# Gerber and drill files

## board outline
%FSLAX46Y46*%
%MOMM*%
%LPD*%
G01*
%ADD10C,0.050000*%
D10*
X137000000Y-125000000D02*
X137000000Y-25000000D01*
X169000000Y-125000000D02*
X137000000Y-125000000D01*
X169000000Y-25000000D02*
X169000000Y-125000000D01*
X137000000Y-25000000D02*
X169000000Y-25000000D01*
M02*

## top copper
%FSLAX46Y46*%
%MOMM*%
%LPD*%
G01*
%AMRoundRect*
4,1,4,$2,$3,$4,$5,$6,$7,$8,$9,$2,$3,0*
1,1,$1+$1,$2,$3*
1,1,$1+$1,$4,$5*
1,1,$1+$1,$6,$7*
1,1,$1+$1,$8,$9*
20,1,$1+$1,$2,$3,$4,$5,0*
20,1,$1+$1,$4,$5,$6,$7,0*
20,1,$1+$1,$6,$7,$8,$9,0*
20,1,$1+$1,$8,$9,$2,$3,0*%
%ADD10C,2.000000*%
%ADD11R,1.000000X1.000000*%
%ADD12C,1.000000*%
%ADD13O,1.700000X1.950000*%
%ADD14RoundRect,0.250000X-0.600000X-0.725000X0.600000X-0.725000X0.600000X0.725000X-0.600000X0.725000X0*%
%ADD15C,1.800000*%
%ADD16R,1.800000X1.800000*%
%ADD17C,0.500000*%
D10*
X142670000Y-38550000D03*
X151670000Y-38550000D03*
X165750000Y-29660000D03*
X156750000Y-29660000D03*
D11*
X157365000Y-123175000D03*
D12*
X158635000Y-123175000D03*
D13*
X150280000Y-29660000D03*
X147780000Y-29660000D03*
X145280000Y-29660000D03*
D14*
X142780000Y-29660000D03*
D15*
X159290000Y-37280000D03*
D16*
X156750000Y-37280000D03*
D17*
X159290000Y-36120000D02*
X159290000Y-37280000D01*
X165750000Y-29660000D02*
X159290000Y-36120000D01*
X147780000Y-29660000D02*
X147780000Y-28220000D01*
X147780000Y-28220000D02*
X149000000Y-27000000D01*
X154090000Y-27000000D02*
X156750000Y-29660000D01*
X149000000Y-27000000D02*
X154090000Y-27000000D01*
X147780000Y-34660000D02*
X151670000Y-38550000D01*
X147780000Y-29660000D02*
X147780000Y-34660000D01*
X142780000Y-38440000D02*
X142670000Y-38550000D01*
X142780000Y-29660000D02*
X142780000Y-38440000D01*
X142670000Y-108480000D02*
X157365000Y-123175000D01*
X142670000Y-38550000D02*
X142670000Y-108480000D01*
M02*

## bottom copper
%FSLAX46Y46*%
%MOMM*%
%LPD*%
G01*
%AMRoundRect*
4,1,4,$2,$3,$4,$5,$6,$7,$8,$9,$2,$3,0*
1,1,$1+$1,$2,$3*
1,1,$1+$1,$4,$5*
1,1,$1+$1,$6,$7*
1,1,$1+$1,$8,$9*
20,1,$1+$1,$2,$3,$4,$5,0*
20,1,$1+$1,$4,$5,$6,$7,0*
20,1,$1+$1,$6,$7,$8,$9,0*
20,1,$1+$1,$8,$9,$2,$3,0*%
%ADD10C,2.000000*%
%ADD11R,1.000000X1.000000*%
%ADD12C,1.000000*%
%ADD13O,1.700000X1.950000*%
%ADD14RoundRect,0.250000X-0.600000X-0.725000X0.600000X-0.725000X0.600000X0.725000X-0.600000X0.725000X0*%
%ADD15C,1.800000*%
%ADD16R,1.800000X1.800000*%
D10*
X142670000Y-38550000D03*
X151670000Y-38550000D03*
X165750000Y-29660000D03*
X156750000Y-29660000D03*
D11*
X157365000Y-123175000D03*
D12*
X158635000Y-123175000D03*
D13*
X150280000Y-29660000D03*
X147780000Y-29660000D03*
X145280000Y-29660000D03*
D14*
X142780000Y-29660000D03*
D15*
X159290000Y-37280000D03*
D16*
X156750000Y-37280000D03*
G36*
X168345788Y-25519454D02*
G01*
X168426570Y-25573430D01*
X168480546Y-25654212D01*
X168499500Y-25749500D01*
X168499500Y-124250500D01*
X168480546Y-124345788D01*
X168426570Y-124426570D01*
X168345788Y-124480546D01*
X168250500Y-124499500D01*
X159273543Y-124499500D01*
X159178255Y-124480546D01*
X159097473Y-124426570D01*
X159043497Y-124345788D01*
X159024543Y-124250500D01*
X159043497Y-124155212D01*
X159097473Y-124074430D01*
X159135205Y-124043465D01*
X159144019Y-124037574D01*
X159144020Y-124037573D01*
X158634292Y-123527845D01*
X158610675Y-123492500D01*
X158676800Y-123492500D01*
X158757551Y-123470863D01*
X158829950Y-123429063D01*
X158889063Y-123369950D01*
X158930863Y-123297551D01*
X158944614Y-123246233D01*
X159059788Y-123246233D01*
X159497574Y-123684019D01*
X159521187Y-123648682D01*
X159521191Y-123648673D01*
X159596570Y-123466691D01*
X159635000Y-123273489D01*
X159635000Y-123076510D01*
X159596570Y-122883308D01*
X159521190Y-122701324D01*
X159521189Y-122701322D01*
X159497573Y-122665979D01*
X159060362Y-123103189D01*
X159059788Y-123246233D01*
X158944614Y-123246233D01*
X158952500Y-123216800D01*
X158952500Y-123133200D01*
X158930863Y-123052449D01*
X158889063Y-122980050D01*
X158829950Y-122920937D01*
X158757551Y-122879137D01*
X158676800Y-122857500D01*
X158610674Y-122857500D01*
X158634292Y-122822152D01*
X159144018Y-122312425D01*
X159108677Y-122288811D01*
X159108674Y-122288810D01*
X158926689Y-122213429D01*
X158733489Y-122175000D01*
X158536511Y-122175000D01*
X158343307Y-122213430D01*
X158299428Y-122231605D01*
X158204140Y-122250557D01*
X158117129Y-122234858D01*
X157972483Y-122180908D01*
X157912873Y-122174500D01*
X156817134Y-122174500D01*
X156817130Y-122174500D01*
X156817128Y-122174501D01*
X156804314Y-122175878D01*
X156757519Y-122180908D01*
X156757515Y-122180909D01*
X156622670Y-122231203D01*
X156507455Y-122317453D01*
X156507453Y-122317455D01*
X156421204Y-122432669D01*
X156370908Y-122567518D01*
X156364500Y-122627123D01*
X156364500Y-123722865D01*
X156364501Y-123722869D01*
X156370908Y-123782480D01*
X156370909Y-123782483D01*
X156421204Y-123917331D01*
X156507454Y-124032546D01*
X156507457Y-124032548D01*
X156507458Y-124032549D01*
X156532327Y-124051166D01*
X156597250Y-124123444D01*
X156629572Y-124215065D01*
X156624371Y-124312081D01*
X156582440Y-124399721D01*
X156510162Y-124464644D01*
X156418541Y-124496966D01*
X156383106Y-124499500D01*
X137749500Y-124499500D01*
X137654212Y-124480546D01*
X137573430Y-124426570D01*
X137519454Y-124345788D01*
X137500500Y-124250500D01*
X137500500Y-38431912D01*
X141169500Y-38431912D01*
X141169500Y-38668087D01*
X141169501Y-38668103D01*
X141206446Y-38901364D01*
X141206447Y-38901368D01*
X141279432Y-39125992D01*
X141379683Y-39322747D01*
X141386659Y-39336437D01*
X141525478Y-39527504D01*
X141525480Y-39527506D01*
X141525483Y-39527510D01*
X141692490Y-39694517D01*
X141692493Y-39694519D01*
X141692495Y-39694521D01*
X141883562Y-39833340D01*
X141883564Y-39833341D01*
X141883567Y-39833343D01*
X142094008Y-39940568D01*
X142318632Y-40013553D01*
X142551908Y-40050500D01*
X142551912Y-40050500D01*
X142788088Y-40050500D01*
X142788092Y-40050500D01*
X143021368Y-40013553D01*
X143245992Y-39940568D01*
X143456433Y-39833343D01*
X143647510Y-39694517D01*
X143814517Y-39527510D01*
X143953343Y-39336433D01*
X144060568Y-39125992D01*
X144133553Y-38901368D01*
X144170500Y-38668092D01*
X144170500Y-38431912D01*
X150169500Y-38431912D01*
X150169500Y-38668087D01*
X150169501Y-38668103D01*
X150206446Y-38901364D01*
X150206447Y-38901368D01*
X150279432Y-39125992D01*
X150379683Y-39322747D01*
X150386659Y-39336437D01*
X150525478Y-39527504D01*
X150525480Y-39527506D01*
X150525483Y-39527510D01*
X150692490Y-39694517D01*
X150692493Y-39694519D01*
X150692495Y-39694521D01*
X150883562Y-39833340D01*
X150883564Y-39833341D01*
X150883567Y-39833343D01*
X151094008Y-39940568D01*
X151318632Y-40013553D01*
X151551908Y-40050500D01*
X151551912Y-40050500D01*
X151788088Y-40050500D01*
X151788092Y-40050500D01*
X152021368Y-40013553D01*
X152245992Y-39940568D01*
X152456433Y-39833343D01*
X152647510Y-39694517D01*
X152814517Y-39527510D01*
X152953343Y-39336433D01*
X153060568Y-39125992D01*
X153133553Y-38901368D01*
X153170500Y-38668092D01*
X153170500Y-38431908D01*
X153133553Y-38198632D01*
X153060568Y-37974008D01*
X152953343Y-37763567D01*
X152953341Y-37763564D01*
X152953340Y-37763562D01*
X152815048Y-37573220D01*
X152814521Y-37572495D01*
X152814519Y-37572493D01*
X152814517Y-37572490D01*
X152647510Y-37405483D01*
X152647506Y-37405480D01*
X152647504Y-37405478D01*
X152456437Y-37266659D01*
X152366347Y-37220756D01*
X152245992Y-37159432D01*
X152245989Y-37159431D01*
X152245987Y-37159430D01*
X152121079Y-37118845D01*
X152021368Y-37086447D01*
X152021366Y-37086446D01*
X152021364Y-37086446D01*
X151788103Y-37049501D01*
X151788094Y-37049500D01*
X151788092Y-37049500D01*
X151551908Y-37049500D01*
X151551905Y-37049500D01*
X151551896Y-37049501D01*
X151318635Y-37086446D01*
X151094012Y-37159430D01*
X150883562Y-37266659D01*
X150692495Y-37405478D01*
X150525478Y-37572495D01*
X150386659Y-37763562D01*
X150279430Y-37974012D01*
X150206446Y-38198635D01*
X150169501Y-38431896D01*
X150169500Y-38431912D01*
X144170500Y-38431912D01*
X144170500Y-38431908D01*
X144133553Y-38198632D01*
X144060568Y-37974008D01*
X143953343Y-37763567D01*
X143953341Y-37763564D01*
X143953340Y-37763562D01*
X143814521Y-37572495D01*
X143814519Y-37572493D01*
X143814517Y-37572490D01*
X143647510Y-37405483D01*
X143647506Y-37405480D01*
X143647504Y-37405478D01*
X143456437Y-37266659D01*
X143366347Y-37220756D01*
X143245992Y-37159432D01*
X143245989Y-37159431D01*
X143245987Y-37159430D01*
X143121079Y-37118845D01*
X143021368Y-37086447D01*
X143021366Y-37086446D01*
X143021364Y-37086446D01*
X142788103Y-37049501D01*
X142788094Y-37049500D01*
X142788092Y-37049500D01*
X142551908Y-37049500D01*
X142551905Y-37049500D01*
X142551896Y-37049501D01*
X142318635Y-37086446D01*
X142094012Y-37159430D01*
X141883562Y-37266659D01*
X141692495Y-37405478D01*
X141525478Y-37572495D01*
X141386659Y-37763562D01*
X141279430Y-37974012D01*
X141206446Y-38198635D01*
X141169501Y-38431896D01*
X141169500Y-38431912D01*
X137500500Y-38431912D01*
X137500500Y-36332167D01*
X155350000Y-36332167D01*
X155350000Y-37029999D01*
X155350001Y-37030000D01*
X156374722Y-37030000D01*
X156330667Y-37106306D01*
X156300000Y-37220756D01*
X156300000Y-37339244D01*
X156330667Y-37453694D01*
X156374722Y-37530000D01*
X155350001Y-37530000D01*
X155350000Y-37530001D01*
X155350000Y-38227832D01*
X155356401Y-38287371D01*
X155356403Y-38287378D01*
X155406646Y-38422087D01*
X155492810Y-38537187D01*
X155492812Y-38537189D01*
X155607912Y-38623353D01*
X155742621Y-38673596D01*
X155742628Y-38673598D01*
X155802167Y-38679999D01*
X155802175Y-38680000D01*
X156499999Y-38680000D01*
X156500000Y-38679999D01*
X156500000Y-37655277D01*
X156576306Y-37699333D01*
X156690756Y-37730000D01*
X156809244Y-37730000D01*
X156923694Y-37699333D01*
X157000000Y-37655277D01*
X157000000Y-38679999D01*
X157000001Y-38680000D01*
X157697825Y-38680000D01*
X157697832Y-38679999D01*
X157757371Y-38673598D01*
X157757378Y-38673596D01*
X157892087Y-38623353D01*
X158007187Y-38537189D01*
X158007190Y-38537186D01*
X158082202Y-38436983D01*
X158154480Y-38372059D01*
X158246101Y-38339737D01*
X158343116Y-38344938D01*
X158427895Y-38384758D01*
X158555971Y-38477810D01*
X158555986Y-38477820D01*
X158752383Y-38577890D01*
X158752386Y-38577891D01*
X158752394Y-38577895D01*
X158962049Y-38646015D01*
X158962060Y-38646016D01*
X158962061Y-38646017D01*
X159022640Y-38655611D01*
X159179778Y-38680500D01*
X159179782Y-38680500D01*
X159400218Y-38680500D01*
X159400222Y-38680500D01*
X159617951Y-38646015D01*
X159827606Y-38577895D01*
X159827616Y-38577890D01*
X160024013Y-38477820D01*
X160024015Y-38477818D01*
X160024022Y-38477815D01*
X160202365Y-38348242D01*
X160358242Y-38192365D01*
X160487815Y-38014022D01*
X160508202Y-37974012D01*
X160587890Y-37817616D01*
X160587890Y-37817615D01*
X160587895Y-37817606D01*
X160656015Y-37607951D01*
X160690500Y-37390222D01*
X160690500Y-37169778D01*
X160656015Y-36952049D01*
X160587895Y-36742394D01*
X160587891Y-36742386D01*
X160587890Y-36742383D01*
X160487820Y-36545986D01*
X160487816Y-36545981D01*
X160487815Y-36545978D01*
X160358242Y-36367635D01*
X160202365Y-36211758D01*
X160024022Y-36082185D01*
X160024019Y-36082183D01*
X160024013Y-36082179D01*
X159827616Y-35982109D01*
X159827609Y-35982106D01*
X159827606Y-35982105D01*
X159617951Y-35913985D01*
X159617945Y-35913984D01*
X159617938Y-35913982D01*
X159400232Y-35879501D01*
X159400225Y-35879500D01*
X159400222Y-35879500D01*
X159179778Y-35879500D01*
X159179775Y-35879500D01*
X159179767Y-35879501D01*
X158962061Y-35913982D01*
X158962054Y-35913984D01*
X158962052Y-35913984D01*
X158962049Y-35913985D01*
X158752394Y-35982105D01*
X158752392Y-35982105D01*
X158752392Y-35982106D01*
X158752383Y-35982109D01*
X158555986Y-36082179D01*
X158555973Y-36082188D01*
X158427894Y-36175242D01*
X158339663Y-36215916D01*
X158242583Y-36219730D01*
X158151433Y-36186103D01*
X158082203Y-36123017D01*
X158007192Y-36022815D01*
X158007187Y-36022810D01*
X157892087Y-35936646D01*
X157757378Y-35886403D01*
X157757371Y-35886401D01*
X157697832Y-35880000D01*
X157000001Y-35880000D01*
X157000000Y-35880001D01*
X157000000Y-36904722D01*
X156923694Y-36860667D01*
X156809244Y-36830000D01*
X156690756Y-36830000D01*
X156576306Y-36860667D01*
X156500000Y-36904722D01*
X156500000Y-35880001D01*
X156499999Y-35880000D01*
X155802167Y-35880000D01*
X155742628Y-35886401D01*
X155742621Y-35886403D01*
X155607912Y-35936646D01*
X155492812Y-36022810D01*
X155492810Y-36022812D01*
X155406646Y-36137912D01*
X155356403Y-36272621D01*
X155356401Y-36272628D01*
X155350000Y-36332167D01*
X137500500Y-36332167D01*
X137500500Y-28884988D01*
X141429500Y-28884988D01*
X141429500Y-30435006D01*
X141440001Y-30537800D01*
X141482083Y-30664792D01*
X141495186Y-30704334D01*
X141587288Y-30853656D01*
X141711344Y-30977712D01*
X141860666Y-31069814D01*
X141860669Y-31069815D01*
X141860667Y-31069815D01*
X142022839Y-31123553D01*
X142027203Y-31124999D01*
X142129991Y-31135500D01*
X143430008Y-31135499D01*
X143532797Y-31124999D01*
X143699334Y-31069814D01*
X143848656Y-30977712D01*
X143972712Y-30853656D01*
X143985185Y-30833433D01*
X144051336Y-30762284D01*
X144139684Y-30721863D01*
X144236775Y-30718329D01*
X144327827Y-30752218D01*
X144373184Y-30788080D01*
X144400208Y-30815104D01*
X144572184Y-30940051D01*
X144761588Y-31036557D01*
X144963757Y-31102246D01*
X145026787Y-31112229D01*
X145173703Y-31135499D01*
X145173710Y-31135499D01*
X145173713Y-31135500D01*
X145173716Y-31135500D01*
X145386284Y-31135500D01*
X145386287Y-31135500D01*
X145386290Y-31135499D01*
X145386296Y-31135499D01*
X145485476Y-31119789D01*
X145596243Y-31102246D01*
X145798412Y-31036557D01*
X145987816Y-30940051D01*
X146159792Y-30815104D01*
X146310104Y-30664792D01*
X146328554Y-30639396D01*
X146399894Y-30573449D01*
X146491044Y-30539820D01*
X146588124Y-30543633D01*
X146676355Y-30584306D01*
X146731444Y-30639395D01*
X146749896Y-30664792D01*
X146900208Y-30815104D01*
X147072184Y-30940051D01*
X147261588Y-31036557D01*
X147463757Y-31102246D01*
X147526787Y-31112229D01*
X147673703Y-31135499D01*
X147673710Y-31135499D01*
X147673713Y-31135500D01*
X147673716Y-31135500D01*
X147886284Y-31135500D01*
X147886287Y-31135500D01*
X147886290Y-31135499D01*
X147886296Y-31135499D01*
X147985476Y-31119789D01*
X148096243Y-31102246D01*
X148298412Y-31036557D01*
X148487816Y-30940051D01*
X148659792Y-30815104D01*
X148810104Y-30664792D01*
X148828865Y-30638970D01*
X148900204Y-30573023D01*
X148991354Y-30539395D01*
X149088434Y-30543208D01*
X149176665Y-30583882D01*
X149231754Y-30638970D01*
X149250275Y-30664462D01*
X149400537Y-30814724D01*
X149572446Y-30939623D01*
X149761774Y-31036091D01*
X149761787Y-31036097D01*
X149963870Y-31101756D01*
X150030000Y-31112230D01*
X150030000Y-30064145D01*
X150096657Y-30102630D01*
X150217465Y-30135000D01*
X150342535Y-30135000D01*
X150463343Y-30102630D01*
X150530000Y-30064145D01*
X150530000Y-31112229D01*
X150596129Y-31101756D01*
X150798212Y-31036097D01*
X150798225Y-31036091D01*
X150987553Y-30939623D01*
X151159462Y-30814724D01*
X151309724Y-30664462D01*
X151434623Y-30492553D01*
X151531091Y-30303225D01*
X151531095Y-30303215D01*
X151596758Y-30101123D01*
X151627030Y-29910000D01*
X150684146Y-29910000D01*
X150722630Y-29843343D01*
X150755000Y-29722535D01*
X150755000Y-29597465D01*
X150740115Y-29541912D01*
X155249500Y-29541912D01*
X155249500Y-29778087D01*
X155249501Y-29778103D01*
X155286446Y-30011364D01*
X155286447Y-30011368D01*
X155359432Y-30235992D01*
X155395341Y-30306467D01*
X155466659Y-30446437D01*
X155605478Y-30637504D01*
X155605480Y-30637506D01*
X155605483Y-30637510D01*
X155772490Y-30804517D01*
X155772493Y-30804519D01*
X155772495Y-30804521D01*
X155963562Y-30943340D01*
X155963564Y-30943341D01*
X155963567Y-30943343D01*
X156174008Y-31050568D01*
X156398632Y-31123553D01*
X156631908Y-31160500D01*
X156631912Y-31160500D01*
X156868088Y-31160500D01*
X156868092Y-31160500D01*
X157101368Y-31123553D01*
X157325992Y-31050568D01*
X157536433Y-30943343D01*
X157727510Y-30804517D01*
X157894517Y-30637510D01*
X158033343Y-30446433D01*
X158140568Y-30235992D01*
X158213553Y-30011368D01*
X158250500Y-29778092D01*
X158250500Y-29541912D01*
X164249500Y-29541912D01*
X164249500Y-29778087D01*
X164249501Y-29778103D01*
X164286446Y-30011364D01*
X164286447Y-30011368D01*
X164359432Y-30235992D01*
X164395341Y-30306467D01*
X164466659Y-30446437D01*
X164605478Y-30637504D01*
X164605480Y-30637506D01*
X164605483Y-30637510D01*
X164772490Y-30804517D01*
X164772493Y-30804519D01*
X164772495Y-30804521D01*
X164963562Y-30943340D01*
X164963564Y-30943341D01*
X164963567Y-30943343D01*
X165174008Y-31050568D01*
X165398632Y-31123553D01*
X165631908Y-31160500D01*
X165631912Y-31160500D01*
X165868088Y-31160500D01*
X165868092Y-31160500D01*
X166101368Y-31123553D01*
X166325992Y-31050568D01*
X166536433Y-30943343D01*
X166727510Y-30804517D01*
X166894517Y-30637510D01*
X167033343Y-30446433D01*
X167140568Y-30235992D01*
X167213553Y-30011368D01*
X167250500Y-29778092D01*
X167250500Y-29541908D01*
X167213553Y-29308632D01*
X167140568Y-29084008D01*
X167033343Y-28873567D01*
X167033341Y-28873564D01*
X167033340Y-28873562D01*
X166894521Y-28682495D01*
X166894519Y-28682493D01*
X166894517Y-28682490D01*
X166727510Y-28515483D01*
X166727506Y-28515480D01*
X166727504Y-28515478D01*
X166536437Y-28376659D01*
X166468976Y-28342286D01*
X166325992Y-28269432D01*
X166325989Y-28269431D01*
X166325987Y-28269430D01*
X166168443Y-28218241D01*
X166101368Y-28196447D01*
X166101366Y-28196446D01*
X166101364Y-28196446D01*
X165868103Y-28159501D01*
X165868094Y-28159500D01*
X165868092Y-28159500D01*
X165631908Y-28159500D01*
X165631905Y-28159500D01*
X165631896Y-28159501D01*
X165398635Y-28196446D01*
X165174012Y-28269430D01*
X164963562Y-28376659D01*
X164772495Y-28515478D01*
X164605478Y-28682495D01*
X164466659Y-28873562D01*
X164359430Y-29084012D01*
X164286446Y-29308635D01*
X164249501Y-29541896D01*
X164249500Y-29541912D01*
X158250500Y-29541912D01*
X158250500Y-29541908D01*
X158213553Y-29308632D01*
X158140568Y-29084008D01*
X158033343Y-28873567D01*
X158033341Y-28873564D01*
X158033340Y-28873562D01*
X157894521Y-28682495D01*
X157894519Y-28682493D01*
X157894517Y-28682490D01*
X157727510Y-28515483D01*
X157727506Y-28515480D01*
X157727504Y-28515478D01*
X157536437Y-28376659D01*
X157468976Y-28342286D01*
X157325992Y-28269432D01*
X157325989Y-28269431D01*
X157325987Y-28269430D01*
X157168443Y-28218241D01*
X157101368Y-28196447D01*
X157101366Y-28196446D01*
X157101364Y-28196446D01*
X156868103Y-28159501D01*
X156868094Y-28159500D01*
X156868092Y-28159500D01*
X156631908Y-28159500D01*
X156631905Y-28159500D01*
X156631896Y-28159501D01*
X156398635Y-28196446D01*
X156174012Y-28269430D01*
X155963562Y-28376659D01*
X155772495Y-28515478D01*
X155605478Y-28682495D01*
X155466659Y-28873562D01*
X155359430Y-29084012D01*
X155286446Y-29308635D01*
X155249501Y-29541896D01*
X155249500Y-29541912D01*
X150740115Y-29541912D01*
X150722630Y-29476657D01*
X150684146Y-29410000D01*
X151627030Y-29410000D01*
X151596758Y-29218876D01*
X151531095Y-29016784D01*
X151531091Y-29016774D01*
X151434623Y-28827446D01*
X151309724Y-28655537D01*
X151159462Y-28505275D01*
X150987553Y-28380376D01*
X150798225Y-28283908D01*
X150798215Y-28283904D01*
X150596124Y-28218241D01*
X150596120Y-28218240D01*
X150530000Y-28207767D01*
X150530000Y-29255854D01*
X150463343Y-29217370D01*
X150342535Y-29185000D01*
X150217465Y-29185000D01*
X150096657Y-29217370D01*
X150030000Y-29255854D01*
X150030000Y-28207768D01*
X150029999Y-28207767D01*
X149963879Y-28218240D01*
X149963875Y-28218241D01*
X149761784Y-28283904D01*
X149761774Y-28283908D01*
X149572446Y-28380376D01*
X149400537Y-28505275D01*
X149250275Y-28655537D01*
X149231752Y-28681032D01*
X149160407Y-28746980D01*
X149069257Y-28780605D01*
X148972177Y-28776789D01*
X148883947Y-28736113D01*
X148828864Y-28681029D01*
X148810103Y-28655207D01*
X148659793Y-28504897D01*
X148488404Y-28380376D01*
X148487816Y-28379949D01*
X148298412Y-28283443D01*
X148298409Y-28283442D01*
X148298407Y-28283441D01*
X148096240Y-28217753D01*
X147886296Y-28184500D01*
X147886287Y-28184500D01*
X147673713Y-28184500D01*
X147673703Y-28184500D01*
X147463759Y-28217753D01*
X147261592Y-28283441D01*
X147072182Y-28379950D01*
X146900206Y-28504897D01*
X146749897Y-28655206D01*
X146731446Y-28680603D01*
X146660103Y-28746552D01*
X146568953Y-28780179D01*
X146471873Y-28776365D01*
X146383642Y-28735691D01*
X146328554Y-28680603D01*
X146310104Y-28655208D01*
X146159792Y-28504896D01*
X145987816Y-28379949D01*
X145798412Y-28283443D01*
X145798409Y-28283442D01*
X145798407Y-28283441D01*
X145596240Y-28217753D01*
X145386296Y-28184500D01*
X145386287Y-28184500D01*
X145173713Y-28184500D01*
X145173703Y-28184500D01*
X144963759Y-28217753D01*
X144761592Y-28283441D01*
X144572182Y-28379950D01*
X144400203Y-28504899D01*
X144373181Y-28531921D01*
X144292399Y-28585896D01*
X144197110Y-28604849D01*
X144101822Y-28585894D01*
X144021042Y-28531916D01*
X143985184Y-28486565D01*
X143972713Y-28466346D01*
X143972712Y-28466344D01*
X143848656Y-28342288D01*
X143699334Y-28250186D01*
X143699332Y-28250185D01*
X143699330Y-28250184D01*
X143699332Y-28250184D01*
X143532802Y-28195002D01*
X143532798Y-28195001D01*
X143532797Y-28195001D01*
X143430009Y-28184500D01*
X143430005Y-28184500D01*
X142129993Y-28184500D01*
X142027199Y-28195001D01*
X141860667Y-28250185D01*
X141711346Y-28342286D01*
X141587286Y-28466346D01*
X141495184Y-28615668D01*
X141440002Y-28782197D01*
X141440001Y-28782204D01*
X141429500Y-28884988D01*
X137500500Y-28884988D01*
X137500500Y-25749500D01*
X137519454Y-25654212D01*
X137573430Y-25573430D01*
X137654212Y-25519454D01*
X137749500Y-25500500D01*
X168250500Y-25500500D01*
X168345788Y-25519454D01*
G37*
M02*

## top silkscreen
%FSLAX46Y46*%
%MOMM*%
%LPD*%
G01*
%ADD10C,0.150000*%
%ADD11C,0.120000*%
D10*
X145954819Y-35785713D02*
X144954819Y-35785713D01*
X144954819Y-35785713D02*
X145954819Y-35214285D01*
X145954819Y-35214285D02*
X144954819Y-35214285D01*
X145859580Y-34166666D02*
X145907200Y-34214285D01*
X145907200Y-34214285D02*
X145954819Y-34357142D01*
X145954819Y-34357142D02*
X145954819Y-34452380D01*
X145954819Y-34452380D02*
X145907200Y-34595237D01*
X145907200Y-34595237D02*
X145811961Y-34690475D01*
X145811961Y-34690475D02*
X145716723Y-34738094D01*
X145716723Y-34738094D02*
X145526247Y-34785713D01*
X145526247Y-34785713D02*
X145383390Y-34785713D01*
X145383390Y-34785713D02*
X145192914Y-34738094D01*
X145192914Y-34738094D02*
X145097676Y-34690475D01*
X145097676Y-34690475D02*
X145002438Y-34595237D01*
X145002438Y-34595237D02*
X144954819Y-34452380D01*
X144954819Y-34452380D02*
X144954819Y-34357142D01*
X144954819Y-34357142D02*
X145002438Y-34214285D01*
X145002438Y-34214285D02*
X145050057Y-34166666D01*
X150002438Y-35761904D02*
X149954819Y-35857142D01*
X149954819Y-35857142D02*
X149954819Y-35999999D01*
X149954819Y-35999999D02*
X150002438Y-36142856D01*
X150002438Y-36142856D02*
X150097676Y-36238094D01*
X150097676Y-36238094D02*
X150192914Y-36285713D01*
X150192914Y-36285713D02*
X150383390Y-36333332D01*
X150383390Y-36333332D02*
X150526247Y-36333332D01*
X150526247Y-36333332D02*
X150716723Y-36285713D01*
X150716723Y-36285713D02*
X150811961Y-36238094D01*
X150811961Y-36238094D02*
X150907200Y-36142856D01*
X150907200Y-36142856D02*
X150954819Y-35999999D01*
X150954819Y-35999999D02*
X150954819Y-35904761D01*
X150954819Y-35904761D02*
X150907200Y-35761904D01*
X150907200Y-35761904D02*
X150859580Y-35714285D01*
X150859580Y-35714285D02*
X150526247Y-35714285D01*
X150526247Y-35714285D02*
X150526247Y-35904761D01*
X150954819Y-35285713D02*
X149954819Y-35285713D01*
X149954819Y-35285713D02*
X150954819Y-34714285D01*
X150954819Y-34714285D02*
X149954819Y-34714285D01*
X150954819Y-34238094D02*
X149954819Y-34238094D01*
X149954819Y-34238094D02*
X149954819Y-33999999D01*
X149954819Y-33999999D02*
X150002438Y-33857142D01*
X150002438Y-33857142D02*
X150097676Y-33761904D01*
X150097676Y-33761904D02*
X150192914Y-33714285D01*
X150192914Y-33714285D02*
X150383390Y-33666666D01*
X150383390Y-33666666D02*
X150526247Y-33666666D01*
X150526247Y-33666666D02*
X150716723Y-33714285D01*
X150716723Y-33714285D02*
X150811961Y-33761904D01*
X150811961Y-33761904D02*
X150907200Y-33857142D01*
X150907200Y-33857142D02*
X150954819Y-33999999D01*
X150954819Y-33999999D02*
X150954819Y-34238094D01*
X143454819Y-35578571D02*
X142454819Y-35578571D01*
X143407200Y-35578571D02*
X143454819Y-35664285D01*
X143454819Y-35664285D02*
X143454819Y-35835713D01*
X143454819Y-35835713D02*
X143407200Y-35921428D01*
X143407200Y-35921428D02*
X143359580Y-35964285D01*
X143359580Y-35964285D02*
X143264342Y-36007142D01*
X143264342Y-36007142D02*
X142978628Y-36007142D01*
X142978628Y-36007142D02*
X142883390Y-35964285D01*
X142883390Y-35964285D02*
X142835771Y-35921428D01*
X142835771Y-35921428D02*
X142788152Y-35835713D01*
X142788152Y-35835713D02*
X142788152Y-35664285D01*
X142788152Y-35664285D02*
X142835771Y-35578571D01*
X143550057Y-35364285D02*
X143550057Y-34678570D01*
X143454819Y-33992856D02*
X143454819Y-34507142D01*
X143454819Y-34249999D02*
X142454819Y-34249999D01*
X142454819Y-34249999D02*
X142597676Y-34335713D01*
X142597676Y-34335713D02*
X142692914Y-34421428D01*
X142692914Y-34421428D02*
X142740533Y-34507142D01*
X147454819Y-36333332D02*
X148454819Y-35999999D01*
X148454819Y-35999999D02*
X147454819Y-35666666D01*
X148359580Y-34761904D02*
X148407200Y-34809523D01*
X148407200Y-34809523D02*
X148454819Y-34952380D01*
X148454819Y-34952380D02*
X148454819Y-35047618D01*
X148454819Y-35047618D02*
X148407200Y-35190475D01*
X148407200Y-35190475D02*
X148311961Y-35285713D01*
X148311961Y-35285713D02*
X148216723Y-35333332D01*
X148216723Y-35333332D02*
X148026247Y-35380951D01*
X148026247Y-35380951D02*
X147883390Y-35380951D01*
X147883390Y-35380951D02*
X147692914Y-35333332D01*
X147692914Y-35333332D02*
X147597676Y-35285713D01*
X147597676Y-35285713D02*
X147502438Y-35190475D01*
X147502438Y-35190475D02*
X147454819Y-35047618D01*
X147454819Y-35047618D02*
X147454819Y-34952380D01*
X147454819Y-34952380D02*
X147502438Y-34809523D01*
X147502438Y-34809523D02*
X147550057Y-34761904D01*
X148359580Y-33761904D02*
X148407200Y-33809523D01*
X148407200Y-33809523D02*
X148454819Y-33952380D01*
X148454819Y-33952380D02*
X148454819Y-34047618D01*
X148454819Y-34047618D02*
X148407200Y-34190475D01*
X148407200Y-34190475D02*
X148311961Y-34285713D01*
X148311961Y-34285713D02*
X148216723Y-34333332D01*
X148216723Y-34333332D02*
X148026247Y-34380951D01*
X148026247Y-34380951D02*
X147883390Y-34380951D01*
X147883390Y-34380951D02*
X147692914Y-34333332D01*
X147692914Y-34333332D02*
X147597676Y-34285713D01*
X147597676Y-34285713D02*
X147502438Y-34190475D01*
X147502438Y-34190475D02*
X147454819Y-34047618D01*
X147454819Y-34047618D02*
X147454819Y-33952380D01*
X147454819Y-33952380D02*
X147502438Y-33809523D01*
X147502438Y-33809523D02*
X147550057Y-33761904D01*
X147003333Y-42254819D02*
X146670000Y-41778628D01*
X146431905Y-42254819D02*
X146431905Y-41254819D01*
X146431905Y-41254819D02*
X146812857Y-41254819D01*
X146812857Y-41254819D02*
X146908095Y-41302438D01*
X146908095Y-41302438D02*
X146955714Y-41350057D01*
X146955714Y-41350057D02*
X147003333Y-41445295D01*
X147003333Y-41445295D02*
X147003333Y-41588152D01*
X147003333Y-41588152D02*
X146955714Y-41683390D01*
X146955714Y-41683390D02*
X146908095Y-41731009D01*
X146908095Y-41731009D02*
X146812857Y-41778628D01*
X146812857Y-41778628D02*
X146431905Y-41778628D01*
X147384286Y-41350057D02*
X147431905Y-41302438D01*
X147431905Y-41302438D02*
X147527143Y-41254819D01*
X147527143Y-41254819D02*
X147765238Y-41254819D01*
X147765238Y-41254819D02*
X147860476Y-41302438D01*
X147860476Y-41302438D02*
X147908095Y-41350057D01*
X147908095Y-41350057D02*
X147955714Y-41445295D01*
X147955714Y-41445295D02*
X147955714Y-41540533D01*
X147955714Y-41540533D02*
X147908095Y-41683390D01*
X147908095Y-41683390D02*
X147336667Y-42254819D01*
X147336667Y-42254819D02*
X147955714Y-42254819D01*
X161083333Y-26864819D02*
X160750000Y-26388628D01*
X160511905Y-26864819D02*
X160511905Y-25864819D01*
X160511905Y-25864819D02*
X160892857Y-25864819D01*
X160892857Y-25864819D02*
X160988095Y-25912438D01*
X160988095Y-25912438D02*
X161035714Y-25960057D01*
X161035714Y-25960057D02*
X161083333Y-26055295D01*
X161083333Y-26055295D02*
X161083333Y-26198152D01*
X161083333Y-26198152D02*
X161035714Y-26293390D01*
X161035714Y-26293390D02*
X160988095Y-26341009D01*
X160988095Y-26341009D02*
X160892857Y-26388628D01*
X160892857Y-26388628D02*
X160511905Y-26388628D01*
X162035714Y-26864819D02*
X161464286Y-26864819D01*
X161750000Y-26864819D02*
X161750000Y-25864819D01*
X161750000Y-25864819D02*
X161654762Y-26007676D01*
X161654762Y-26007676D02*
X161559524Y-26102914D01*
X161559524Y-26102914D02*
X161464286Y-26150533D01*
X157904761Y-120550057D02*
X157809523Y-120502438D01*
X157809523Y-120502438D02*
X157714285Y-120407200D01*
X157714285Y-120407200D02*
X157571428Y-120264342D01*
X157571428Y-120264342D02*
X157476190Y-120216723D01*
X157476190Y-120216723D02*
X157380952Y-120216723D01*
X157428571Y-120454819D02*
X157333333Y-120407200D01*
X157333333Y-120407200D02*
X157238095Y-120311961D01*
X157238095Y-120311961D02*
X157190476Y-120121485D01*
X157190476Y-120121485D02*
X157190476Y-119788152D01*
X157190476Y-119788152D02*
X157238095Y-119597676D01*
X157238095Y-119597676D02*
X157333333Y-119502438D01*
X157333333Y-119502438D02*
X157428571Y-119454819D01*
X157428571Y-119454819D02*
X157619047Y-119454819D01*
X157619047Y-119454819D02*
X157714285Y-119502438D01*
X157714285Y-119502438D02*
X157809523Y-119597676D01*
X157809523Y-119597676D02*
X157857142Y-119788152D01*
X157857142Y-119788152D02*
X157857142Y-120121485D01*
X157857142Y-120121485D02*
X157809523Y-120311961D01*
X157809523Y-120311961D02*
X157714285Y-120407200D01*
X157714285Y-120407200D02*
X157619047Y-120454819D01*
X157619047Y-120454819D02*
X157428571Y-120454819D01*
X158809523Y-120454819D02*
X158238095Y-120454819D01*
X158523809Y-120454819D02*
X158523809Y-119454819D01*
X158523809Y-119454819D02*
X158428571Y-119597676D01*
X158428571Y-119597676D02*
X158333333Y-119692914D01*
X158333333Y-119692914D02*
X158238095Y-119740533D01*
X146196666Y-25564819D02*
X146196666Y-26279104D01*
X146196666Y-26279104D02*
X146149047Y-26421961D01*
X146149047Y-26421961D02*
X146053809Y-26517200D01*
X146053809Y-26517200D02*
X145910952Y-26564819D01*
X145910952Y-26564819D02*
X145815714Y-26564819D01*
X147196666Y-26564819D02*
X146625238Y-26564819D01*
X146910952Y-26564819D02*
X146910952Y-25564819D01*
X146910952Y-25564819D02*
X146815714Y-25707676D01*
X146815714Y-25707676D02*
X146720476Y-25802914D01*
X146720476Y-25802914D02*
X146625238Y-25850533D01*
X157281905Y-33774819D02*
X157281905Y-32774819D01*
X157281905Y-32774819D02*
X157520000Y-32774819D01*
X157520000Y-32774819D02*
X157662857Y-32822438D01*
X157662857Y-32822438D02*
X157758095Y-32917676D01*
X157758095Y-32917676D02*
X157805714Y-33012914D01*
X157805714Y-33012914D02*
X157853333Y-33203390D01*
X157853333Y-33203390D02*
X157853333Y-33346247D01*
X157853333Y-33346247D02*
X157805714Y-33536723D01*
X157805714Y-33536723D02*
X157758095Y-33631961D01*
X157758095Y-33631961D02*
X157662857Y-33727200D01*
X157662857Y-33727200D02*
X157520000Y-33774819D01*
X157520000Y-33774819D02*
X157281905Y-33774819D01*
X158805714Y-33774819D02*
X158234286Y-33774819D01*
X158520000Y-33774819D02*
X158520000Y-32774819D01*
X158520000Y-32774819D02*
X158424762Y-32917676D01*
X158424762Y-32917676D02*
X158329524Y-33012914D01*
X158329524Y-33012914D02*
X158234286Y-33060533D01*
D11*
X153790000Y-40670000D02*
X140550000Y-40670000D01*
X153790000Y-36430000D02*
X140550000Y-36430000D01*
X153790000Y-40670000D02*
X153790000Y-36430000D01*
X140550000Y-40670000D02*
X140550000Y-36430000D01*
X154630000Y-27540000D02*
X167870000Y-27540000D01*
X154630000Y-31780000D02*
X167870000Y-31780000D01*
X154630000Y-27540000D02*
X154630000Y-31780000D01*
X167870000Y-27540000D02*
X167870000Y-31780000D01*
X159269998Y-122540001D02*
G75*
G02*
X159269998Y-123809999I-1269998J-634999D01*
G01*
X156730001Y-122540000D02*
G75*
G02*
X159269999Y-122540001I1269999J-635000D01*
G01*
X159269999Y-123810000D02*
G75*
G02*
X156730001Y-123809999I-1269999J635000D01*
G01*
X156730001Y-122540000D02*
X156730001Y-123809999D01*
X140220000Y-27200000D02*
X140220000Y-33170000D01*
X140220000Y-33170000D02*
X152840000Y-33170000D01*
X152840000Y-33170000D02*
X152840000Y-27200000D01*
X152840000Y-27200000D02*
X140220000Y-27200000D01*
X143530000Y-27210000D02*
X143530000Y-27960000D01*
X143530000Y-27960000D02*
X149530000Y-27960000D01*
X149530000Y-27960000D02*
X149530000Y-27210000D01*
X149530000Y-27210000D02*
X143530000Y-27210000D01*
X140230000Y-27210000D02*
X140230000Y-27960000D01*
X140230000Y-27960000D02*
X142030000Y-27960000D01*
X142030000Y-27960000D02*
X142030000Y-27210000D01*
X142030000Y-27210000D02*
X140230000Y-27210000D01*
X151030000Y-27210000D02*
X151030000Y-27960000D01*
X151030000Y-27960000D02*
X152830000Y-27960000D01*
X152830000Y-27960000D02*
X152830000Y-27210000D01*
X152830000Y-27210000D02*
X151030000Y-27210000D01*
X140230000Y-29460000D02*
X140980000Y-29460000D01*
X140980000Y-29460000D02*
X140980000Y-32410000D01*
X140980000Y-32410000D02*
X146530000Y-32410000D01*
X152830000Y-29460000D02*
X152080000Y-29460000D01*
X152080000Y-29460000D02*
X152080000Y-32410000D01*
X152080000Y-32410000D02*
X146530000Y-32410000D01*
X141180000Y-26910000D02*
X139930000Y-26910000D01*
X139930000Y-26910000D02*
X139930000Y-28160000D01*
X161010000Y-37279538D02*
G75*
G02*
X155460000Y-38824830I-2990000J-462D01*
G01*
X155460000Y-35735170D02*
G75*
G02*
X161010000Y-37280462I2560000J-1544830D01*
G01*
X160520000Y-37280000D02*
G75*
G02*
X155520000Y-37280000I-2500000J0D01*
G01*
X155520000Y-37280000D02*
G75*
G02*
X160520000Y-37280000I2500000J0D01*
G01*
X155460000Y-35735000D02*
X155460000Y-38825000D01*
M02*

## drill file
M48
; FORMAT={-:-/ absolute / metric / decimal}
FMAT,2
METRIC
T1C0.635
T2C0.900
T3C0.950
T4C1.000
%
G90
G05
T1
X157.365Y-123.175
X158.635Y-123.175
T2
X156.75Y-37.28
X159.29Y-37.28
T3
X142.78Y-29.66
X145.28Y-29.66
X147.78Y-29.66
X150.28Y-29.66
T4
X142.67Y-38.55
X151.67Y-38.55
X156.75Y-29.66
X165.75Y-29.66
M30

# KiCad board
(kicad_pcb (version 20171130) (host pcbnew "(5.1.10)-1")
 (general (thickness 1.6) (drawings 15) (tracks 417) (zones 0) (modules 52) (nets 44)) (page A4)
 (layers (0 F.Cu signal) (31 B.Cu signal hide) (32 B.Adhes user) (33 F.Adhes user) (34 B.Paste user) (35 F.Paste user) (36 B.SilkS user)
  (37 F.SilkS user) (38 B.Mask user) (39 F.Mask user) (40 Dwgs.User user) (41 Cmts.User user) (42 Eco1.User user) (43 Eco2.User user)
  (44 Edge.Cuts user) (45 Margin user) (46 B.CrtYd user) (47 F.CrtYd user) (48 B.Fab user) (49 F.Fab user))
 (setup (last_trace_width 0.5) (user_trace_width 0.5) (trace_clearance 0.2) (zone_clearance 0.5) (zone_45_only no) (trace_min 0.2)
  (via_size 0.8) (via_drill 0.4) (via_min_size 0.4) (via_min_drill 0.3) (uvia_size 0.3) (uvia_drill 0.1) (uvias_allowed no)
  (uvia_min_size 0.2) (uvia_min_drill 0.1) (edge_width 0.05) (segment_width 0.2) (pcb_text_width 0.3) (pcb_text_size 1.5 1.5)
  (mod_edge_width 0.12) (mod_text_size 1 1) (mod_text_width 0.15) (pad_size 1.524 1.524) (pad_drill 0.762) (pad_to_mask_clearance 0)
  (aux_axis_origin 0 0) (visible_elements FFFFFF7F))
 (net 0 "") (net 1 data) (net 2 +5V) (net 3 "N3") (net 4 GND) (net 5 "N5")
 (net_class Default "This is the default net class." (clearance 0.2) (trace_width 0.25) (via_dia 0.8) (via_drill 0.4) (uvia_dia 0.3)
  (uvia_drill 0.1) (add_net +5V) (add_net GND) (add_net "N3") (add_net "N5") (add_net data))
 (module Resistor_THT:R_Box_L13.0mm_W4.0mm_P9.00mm (layer F.Cu) (at 151.67 38.55 180)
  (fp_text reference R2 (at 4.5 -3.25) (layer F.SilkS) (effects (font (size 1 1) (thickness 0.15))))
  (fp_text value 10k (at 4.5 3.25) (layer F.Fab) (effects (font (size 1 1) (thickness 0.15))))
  (fp_line (start -2.12 -2.12) (end 11.12 -2.12) (layer F.SilkS) (width 0.12))
  (fp_line (start -2.12 2.12) (end 11.12 2.12) (layer F.SilkS) (width 0.12))
  (fp_line (start -2.12 -2.12) (end -2.12 2.12) (layer F.SilkS) (width 0.12))
  (fp_line (start 11.12 -2.12) (end 11.12 2.12) (layer F.SilkS) (width 0.12))
  (pad 2 thru_hole circle (at 9 0 180) (size 2 2) (drill 1) (layers *.Cu *.Mask) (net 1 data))
  (pad 1 thru_hole circle (at 0 0 180) (size 2 2) (drill 1) (layers *.Cu *.Mask) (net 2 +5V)))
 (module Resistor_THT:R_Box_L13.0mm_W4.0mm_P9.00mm (layer F.Cu) (at 156.75 29.66)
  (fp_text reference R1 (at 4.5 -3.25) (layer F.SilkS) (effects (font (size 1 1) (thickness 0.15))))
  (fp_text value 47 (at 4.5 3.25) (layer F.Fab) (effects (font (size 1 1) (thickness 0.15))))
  (fp_line (start -2.12 -2.12) (end 11.12 -2.12) (layer F.SilkS) (width 0.12))
  (fp_line (start -2.12 2.12) (end 11.12 2.12) (layer F.SilkS) (width 0.12))
  (fp_line (start -2.12 -2.12) (end -2.12 2.12) (layer F.SilkS) (width 0.12))
  (fp_line (start 11.12 -2.12) (end 11.12 2.12) (layer F.SilkS) (width 0.12))
  (pad 2 thru_hole circle (at 9 0) (size 2 2) (drill 1) (layers *.Cu *.Mask) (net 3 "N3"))
  (pad 1 thru_hole circle (at 0 0) (size 2 2) (drill 1) (layers *.Cu *.Mask) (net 2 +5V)))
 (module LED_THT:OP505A (layer F.Cu) (at 158 120)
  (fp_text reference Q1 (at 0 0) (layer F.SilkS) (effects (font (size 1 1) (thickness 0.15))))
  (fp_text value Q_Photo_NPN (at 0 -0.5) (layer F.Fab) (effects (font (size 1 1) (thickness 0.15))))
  (fp_arc (start 0 3.175) (end 1.269998 3.809999) (angle -53.13010235) (layer F.SilkS) (width 0.12))
  (fp_arc (start 0 3.175) (end 1.269999 2.540001) (angle -126.8698976) (layer F.SilkS) (width 0.12))
  (fp_arc (start 0 3.175) (end -1.269999 3.809999) (angle -126.8698976) (layer F.SilkS) (width 0.12))
  (fp_line (start -1.269999 2.54) (end -1.269999 3.809999) (layer F.SilkS) (width 0.12))
  (pad 1 thru_hole rect (at -0.635 3.175) (size 1 1) (drill 0.635) (layers *.Cu *.Mask) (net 1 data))
  (pad 2 thru_hole circle (at 0.635 3.175) (size 1 1) (drill 0.635) (layers *.Cu *.Mask) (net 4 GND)))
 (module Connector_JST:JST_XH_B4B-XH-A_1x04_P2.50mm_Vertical (layer F.Cu) (at 142.78 29.66)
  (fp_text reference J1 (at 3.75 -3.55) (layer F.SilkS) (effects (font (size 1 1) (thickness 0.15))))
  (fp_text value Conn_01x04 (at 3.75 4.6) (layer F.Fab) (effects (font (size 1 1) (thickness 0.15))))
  (fp_line (start -2.56 -2.46) (end -2.56 3.51) (layer F.SilkS) (width 0.12))
  (fp_line (start -2.56 3.51) (end 10.06 3.51) (layer F.SilkS) (width 0.12))
  (fp_line (start 10.06 3.51) (end 10.06 -2.46) (layer F.SilkS) (width 0.12))
  (fp_line (start 10.06 -2.46) (end -2.56 -2.46) (layer F.SilkS) (width 0.12))
  (fp_line (start 0.75 -2.45) (end 0.75 -1.7) (layer F.SilkS) (width 0.12))
  (fp_line (start 0.75 -1.7) (end 6.75 -1.7) (layer F.SilkS) (width 0.12))
  (fp_line (start 6.75 -1.7) (end 6.75 -2.45) (layer F.SilkS) (width 0.12))
  (fp_line (start 6.75 -2.45) (end 0.75 -2.45) (layer F.SilkS) (width 0.12))
  (fp_line (start -2.55 -2.45) (end -2.55 -1.7) (layer F.SilkS) (width 0.12))
  (fp_line (start -2.55 -1.7) (end -0.75 -1.7) (layer F.SilkS) (width 0.12))
  (fp_line (start -0.75 -1.7) (end -0.75 -2.45) (layer F.SilkS) (width 0.12))
  (fp_line (start -0.75 -2.45) (end -2.55 -2.45) (layer F.SilkS) (width 0.12))
  (fp_line (start 8.25 -2.45) (end 8.25 -1.7) (layer F.SilkS) (width 0.12))
  (fp_line (start 8.25 -1.7) (end 10.05 -1.7) (layer F.SilkS) (width 0.12))
  (fp_line (start 10.05 -1.7) (end 10.05 -2.45) (layer F.SilkS) (width 0.12))
  (fp_line (start 10.05 -2.45) (end 8.25 -2.45) (layer F.SilkS) (width 0.12))
  (fp_line (start -2.55 -0.2) (end -1.8 -0.2) (layer F.SilkS) (width 0.12))
  (fp_line (start -1.8 -0.2) (end -1.8 2.75) (layer F.SilkS) (width 0.12))
  (fp_line (start -1.8 2.75) (end 3.75 2.75) (layer F.SilkS) (width 0.12))
  (fp_line (start 10.05 -0.2) (end 9.3 -0.2) (layer F.SilkS) (width 0.12))
  (fp_line (start 9.3 -0.2) (end 9.3 2.75) (layer F.SilkS) (width 0.12))
  (fp_line (start 9.3 2.75) (end 3.75 2.75) (layer F.SilkS) (width 0.12))
  (fp_line (start -1.6 -2.75) (end -2.85 -2.75) (layer F.SilkS) (width 0.12))
  (fp_line (start -2.85 -2.75) (end -2.85 -1.5) (layer F.SilkS) (width 0.12))
  (pad 4 thru_hole oval (at 7.5 0) (size 1.7 1.95) (drill 0.95) (layers *.Cu *.Mask) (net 4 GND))
  (pad 3 thru_hole oval (at 5 0) (size 1.7 1.95) (drill 0.95) (layers *.Cu *.Mask) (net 2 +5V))
  (pad 2 thru_hole oval (at 2.5 0) (size 1.7 1.95) (drill 0.95) (layers *.Cu *.Mask) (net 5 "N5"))
  (pad 1 thru_hole roundrect (at 0 0) (size 1.7 1.95) (drill 0.95) (layers *.Cu *.Mask) (roundrect_rratio 0.1470588235294118) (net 1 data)))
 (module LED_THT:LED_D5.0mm (layer F.Cu) (at 156.75 37.28)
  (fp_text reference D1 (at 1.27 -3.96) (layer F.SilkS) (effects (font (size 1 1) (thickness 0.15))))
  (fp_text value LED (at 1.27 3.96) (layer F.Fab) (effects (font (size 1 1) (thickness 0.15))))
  (fp_arc (start 1.27 0) (end -1.29 1.54483) (angle -148.9) (layer F.SilkS) (width 0.12))
  (fp_arc (start 1.27 0) (end -1.29 -1.54483) (angle 148.9) (layer F.SilkS) (width 0.12))
  (fp_circle (center 1.27 0) (end 3.77 0) (layer F.SilkS) (width 0.12))
  (fp_line (start -1.29 -1.545) (end -1.29 1.545) (layer F.SilkS) (width 0.12))
  (pad 2 thru_hole circle (at 2.54 0) (size 1.8 1.8) (drill 0.9) (layers *.Cu *.Mask) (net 3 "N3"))
  (pad 1 thru_hole rect (at 0 0) (size 1.8 1.8) (drill 0.9) (layers *.Cu *.Mask) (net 4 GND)))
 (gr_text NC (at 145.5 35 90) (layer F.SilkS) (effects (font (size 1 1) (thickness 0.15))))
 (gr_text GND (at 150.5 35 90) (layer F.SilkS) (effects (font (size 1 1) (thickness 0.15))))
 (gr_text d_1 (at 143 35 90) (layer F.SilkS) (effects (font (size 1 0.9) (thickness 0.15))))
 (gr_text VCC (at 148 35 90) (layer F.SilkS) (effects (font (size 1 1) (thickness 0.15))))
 (gr_line (start 137 125) (end 137 25) (layer Edge.Cuts) (width 0.05))
 (gr_line (start 169 125) (end 137 125) (layer Edge.Cuts) (width 0.05))
 (gr_line (start 169 25) (end 169 125) (layer Edge.Cuts) (width 0.05))
 (gr_line (start 137 25) (end 169 25) (layer Edge.Cuts) (width 0.05))
 (segment (start 159.29 36.12) (end 159.29 37.28) (width 0.5) (layer F.Cu) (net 3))
 (segment (start 165.75 29.66) (end 159.29 36.12) (width 0.5) (layer F.Cu) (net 3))
 (segment (start 147.78 29.66) (end 147.78 28.22) (width 0.5) (layer F.Cu) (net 2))
 (segment (start 147.78 28.22) (end 149 27) (width 0.5) (layer F.Cu) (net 2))
 (segment (start 154.09 27) (end 156.75 29.66) (width 0.5) (layer F.Cu) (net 2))
 (segment (start 149 27) (end 154.09 27) (width 0.5) (layer F.Cu) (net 2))
 (segment (start 147.78 34.66) (end 151.67 38.55) (width 0.5) (layer F.Cu) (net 2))
 (segment (start 147.78 29.66) (end 147.78 34.66) (width 0.5) (layer F.Cu) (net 2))
 (segment (start 142.78 38.44) (end 142.67 38.55) (width 0.5) (layer F.Cu) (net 1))
 (segment (start 142.78 29.66) (end 142.78 38.44) (width 0.5) (layer F.Cu) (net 1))
 (segment (start 142.67 108.48) (end 157.365 123.175) (width 0.5) (layer F.Cu) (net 1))
 (segment (start 142.67 38.55) (end 142.67 108.48) (width 0.5) (layer F.Cu) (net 1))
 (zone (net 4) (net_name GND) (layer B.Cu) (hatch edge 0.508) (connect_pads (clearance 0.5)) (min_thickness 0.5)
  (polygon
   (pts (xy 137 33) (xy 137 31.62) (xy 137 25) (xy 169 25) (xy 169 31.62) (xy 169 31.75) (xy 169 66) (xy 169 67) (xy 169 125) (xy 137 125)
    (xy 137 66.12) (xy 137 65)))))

